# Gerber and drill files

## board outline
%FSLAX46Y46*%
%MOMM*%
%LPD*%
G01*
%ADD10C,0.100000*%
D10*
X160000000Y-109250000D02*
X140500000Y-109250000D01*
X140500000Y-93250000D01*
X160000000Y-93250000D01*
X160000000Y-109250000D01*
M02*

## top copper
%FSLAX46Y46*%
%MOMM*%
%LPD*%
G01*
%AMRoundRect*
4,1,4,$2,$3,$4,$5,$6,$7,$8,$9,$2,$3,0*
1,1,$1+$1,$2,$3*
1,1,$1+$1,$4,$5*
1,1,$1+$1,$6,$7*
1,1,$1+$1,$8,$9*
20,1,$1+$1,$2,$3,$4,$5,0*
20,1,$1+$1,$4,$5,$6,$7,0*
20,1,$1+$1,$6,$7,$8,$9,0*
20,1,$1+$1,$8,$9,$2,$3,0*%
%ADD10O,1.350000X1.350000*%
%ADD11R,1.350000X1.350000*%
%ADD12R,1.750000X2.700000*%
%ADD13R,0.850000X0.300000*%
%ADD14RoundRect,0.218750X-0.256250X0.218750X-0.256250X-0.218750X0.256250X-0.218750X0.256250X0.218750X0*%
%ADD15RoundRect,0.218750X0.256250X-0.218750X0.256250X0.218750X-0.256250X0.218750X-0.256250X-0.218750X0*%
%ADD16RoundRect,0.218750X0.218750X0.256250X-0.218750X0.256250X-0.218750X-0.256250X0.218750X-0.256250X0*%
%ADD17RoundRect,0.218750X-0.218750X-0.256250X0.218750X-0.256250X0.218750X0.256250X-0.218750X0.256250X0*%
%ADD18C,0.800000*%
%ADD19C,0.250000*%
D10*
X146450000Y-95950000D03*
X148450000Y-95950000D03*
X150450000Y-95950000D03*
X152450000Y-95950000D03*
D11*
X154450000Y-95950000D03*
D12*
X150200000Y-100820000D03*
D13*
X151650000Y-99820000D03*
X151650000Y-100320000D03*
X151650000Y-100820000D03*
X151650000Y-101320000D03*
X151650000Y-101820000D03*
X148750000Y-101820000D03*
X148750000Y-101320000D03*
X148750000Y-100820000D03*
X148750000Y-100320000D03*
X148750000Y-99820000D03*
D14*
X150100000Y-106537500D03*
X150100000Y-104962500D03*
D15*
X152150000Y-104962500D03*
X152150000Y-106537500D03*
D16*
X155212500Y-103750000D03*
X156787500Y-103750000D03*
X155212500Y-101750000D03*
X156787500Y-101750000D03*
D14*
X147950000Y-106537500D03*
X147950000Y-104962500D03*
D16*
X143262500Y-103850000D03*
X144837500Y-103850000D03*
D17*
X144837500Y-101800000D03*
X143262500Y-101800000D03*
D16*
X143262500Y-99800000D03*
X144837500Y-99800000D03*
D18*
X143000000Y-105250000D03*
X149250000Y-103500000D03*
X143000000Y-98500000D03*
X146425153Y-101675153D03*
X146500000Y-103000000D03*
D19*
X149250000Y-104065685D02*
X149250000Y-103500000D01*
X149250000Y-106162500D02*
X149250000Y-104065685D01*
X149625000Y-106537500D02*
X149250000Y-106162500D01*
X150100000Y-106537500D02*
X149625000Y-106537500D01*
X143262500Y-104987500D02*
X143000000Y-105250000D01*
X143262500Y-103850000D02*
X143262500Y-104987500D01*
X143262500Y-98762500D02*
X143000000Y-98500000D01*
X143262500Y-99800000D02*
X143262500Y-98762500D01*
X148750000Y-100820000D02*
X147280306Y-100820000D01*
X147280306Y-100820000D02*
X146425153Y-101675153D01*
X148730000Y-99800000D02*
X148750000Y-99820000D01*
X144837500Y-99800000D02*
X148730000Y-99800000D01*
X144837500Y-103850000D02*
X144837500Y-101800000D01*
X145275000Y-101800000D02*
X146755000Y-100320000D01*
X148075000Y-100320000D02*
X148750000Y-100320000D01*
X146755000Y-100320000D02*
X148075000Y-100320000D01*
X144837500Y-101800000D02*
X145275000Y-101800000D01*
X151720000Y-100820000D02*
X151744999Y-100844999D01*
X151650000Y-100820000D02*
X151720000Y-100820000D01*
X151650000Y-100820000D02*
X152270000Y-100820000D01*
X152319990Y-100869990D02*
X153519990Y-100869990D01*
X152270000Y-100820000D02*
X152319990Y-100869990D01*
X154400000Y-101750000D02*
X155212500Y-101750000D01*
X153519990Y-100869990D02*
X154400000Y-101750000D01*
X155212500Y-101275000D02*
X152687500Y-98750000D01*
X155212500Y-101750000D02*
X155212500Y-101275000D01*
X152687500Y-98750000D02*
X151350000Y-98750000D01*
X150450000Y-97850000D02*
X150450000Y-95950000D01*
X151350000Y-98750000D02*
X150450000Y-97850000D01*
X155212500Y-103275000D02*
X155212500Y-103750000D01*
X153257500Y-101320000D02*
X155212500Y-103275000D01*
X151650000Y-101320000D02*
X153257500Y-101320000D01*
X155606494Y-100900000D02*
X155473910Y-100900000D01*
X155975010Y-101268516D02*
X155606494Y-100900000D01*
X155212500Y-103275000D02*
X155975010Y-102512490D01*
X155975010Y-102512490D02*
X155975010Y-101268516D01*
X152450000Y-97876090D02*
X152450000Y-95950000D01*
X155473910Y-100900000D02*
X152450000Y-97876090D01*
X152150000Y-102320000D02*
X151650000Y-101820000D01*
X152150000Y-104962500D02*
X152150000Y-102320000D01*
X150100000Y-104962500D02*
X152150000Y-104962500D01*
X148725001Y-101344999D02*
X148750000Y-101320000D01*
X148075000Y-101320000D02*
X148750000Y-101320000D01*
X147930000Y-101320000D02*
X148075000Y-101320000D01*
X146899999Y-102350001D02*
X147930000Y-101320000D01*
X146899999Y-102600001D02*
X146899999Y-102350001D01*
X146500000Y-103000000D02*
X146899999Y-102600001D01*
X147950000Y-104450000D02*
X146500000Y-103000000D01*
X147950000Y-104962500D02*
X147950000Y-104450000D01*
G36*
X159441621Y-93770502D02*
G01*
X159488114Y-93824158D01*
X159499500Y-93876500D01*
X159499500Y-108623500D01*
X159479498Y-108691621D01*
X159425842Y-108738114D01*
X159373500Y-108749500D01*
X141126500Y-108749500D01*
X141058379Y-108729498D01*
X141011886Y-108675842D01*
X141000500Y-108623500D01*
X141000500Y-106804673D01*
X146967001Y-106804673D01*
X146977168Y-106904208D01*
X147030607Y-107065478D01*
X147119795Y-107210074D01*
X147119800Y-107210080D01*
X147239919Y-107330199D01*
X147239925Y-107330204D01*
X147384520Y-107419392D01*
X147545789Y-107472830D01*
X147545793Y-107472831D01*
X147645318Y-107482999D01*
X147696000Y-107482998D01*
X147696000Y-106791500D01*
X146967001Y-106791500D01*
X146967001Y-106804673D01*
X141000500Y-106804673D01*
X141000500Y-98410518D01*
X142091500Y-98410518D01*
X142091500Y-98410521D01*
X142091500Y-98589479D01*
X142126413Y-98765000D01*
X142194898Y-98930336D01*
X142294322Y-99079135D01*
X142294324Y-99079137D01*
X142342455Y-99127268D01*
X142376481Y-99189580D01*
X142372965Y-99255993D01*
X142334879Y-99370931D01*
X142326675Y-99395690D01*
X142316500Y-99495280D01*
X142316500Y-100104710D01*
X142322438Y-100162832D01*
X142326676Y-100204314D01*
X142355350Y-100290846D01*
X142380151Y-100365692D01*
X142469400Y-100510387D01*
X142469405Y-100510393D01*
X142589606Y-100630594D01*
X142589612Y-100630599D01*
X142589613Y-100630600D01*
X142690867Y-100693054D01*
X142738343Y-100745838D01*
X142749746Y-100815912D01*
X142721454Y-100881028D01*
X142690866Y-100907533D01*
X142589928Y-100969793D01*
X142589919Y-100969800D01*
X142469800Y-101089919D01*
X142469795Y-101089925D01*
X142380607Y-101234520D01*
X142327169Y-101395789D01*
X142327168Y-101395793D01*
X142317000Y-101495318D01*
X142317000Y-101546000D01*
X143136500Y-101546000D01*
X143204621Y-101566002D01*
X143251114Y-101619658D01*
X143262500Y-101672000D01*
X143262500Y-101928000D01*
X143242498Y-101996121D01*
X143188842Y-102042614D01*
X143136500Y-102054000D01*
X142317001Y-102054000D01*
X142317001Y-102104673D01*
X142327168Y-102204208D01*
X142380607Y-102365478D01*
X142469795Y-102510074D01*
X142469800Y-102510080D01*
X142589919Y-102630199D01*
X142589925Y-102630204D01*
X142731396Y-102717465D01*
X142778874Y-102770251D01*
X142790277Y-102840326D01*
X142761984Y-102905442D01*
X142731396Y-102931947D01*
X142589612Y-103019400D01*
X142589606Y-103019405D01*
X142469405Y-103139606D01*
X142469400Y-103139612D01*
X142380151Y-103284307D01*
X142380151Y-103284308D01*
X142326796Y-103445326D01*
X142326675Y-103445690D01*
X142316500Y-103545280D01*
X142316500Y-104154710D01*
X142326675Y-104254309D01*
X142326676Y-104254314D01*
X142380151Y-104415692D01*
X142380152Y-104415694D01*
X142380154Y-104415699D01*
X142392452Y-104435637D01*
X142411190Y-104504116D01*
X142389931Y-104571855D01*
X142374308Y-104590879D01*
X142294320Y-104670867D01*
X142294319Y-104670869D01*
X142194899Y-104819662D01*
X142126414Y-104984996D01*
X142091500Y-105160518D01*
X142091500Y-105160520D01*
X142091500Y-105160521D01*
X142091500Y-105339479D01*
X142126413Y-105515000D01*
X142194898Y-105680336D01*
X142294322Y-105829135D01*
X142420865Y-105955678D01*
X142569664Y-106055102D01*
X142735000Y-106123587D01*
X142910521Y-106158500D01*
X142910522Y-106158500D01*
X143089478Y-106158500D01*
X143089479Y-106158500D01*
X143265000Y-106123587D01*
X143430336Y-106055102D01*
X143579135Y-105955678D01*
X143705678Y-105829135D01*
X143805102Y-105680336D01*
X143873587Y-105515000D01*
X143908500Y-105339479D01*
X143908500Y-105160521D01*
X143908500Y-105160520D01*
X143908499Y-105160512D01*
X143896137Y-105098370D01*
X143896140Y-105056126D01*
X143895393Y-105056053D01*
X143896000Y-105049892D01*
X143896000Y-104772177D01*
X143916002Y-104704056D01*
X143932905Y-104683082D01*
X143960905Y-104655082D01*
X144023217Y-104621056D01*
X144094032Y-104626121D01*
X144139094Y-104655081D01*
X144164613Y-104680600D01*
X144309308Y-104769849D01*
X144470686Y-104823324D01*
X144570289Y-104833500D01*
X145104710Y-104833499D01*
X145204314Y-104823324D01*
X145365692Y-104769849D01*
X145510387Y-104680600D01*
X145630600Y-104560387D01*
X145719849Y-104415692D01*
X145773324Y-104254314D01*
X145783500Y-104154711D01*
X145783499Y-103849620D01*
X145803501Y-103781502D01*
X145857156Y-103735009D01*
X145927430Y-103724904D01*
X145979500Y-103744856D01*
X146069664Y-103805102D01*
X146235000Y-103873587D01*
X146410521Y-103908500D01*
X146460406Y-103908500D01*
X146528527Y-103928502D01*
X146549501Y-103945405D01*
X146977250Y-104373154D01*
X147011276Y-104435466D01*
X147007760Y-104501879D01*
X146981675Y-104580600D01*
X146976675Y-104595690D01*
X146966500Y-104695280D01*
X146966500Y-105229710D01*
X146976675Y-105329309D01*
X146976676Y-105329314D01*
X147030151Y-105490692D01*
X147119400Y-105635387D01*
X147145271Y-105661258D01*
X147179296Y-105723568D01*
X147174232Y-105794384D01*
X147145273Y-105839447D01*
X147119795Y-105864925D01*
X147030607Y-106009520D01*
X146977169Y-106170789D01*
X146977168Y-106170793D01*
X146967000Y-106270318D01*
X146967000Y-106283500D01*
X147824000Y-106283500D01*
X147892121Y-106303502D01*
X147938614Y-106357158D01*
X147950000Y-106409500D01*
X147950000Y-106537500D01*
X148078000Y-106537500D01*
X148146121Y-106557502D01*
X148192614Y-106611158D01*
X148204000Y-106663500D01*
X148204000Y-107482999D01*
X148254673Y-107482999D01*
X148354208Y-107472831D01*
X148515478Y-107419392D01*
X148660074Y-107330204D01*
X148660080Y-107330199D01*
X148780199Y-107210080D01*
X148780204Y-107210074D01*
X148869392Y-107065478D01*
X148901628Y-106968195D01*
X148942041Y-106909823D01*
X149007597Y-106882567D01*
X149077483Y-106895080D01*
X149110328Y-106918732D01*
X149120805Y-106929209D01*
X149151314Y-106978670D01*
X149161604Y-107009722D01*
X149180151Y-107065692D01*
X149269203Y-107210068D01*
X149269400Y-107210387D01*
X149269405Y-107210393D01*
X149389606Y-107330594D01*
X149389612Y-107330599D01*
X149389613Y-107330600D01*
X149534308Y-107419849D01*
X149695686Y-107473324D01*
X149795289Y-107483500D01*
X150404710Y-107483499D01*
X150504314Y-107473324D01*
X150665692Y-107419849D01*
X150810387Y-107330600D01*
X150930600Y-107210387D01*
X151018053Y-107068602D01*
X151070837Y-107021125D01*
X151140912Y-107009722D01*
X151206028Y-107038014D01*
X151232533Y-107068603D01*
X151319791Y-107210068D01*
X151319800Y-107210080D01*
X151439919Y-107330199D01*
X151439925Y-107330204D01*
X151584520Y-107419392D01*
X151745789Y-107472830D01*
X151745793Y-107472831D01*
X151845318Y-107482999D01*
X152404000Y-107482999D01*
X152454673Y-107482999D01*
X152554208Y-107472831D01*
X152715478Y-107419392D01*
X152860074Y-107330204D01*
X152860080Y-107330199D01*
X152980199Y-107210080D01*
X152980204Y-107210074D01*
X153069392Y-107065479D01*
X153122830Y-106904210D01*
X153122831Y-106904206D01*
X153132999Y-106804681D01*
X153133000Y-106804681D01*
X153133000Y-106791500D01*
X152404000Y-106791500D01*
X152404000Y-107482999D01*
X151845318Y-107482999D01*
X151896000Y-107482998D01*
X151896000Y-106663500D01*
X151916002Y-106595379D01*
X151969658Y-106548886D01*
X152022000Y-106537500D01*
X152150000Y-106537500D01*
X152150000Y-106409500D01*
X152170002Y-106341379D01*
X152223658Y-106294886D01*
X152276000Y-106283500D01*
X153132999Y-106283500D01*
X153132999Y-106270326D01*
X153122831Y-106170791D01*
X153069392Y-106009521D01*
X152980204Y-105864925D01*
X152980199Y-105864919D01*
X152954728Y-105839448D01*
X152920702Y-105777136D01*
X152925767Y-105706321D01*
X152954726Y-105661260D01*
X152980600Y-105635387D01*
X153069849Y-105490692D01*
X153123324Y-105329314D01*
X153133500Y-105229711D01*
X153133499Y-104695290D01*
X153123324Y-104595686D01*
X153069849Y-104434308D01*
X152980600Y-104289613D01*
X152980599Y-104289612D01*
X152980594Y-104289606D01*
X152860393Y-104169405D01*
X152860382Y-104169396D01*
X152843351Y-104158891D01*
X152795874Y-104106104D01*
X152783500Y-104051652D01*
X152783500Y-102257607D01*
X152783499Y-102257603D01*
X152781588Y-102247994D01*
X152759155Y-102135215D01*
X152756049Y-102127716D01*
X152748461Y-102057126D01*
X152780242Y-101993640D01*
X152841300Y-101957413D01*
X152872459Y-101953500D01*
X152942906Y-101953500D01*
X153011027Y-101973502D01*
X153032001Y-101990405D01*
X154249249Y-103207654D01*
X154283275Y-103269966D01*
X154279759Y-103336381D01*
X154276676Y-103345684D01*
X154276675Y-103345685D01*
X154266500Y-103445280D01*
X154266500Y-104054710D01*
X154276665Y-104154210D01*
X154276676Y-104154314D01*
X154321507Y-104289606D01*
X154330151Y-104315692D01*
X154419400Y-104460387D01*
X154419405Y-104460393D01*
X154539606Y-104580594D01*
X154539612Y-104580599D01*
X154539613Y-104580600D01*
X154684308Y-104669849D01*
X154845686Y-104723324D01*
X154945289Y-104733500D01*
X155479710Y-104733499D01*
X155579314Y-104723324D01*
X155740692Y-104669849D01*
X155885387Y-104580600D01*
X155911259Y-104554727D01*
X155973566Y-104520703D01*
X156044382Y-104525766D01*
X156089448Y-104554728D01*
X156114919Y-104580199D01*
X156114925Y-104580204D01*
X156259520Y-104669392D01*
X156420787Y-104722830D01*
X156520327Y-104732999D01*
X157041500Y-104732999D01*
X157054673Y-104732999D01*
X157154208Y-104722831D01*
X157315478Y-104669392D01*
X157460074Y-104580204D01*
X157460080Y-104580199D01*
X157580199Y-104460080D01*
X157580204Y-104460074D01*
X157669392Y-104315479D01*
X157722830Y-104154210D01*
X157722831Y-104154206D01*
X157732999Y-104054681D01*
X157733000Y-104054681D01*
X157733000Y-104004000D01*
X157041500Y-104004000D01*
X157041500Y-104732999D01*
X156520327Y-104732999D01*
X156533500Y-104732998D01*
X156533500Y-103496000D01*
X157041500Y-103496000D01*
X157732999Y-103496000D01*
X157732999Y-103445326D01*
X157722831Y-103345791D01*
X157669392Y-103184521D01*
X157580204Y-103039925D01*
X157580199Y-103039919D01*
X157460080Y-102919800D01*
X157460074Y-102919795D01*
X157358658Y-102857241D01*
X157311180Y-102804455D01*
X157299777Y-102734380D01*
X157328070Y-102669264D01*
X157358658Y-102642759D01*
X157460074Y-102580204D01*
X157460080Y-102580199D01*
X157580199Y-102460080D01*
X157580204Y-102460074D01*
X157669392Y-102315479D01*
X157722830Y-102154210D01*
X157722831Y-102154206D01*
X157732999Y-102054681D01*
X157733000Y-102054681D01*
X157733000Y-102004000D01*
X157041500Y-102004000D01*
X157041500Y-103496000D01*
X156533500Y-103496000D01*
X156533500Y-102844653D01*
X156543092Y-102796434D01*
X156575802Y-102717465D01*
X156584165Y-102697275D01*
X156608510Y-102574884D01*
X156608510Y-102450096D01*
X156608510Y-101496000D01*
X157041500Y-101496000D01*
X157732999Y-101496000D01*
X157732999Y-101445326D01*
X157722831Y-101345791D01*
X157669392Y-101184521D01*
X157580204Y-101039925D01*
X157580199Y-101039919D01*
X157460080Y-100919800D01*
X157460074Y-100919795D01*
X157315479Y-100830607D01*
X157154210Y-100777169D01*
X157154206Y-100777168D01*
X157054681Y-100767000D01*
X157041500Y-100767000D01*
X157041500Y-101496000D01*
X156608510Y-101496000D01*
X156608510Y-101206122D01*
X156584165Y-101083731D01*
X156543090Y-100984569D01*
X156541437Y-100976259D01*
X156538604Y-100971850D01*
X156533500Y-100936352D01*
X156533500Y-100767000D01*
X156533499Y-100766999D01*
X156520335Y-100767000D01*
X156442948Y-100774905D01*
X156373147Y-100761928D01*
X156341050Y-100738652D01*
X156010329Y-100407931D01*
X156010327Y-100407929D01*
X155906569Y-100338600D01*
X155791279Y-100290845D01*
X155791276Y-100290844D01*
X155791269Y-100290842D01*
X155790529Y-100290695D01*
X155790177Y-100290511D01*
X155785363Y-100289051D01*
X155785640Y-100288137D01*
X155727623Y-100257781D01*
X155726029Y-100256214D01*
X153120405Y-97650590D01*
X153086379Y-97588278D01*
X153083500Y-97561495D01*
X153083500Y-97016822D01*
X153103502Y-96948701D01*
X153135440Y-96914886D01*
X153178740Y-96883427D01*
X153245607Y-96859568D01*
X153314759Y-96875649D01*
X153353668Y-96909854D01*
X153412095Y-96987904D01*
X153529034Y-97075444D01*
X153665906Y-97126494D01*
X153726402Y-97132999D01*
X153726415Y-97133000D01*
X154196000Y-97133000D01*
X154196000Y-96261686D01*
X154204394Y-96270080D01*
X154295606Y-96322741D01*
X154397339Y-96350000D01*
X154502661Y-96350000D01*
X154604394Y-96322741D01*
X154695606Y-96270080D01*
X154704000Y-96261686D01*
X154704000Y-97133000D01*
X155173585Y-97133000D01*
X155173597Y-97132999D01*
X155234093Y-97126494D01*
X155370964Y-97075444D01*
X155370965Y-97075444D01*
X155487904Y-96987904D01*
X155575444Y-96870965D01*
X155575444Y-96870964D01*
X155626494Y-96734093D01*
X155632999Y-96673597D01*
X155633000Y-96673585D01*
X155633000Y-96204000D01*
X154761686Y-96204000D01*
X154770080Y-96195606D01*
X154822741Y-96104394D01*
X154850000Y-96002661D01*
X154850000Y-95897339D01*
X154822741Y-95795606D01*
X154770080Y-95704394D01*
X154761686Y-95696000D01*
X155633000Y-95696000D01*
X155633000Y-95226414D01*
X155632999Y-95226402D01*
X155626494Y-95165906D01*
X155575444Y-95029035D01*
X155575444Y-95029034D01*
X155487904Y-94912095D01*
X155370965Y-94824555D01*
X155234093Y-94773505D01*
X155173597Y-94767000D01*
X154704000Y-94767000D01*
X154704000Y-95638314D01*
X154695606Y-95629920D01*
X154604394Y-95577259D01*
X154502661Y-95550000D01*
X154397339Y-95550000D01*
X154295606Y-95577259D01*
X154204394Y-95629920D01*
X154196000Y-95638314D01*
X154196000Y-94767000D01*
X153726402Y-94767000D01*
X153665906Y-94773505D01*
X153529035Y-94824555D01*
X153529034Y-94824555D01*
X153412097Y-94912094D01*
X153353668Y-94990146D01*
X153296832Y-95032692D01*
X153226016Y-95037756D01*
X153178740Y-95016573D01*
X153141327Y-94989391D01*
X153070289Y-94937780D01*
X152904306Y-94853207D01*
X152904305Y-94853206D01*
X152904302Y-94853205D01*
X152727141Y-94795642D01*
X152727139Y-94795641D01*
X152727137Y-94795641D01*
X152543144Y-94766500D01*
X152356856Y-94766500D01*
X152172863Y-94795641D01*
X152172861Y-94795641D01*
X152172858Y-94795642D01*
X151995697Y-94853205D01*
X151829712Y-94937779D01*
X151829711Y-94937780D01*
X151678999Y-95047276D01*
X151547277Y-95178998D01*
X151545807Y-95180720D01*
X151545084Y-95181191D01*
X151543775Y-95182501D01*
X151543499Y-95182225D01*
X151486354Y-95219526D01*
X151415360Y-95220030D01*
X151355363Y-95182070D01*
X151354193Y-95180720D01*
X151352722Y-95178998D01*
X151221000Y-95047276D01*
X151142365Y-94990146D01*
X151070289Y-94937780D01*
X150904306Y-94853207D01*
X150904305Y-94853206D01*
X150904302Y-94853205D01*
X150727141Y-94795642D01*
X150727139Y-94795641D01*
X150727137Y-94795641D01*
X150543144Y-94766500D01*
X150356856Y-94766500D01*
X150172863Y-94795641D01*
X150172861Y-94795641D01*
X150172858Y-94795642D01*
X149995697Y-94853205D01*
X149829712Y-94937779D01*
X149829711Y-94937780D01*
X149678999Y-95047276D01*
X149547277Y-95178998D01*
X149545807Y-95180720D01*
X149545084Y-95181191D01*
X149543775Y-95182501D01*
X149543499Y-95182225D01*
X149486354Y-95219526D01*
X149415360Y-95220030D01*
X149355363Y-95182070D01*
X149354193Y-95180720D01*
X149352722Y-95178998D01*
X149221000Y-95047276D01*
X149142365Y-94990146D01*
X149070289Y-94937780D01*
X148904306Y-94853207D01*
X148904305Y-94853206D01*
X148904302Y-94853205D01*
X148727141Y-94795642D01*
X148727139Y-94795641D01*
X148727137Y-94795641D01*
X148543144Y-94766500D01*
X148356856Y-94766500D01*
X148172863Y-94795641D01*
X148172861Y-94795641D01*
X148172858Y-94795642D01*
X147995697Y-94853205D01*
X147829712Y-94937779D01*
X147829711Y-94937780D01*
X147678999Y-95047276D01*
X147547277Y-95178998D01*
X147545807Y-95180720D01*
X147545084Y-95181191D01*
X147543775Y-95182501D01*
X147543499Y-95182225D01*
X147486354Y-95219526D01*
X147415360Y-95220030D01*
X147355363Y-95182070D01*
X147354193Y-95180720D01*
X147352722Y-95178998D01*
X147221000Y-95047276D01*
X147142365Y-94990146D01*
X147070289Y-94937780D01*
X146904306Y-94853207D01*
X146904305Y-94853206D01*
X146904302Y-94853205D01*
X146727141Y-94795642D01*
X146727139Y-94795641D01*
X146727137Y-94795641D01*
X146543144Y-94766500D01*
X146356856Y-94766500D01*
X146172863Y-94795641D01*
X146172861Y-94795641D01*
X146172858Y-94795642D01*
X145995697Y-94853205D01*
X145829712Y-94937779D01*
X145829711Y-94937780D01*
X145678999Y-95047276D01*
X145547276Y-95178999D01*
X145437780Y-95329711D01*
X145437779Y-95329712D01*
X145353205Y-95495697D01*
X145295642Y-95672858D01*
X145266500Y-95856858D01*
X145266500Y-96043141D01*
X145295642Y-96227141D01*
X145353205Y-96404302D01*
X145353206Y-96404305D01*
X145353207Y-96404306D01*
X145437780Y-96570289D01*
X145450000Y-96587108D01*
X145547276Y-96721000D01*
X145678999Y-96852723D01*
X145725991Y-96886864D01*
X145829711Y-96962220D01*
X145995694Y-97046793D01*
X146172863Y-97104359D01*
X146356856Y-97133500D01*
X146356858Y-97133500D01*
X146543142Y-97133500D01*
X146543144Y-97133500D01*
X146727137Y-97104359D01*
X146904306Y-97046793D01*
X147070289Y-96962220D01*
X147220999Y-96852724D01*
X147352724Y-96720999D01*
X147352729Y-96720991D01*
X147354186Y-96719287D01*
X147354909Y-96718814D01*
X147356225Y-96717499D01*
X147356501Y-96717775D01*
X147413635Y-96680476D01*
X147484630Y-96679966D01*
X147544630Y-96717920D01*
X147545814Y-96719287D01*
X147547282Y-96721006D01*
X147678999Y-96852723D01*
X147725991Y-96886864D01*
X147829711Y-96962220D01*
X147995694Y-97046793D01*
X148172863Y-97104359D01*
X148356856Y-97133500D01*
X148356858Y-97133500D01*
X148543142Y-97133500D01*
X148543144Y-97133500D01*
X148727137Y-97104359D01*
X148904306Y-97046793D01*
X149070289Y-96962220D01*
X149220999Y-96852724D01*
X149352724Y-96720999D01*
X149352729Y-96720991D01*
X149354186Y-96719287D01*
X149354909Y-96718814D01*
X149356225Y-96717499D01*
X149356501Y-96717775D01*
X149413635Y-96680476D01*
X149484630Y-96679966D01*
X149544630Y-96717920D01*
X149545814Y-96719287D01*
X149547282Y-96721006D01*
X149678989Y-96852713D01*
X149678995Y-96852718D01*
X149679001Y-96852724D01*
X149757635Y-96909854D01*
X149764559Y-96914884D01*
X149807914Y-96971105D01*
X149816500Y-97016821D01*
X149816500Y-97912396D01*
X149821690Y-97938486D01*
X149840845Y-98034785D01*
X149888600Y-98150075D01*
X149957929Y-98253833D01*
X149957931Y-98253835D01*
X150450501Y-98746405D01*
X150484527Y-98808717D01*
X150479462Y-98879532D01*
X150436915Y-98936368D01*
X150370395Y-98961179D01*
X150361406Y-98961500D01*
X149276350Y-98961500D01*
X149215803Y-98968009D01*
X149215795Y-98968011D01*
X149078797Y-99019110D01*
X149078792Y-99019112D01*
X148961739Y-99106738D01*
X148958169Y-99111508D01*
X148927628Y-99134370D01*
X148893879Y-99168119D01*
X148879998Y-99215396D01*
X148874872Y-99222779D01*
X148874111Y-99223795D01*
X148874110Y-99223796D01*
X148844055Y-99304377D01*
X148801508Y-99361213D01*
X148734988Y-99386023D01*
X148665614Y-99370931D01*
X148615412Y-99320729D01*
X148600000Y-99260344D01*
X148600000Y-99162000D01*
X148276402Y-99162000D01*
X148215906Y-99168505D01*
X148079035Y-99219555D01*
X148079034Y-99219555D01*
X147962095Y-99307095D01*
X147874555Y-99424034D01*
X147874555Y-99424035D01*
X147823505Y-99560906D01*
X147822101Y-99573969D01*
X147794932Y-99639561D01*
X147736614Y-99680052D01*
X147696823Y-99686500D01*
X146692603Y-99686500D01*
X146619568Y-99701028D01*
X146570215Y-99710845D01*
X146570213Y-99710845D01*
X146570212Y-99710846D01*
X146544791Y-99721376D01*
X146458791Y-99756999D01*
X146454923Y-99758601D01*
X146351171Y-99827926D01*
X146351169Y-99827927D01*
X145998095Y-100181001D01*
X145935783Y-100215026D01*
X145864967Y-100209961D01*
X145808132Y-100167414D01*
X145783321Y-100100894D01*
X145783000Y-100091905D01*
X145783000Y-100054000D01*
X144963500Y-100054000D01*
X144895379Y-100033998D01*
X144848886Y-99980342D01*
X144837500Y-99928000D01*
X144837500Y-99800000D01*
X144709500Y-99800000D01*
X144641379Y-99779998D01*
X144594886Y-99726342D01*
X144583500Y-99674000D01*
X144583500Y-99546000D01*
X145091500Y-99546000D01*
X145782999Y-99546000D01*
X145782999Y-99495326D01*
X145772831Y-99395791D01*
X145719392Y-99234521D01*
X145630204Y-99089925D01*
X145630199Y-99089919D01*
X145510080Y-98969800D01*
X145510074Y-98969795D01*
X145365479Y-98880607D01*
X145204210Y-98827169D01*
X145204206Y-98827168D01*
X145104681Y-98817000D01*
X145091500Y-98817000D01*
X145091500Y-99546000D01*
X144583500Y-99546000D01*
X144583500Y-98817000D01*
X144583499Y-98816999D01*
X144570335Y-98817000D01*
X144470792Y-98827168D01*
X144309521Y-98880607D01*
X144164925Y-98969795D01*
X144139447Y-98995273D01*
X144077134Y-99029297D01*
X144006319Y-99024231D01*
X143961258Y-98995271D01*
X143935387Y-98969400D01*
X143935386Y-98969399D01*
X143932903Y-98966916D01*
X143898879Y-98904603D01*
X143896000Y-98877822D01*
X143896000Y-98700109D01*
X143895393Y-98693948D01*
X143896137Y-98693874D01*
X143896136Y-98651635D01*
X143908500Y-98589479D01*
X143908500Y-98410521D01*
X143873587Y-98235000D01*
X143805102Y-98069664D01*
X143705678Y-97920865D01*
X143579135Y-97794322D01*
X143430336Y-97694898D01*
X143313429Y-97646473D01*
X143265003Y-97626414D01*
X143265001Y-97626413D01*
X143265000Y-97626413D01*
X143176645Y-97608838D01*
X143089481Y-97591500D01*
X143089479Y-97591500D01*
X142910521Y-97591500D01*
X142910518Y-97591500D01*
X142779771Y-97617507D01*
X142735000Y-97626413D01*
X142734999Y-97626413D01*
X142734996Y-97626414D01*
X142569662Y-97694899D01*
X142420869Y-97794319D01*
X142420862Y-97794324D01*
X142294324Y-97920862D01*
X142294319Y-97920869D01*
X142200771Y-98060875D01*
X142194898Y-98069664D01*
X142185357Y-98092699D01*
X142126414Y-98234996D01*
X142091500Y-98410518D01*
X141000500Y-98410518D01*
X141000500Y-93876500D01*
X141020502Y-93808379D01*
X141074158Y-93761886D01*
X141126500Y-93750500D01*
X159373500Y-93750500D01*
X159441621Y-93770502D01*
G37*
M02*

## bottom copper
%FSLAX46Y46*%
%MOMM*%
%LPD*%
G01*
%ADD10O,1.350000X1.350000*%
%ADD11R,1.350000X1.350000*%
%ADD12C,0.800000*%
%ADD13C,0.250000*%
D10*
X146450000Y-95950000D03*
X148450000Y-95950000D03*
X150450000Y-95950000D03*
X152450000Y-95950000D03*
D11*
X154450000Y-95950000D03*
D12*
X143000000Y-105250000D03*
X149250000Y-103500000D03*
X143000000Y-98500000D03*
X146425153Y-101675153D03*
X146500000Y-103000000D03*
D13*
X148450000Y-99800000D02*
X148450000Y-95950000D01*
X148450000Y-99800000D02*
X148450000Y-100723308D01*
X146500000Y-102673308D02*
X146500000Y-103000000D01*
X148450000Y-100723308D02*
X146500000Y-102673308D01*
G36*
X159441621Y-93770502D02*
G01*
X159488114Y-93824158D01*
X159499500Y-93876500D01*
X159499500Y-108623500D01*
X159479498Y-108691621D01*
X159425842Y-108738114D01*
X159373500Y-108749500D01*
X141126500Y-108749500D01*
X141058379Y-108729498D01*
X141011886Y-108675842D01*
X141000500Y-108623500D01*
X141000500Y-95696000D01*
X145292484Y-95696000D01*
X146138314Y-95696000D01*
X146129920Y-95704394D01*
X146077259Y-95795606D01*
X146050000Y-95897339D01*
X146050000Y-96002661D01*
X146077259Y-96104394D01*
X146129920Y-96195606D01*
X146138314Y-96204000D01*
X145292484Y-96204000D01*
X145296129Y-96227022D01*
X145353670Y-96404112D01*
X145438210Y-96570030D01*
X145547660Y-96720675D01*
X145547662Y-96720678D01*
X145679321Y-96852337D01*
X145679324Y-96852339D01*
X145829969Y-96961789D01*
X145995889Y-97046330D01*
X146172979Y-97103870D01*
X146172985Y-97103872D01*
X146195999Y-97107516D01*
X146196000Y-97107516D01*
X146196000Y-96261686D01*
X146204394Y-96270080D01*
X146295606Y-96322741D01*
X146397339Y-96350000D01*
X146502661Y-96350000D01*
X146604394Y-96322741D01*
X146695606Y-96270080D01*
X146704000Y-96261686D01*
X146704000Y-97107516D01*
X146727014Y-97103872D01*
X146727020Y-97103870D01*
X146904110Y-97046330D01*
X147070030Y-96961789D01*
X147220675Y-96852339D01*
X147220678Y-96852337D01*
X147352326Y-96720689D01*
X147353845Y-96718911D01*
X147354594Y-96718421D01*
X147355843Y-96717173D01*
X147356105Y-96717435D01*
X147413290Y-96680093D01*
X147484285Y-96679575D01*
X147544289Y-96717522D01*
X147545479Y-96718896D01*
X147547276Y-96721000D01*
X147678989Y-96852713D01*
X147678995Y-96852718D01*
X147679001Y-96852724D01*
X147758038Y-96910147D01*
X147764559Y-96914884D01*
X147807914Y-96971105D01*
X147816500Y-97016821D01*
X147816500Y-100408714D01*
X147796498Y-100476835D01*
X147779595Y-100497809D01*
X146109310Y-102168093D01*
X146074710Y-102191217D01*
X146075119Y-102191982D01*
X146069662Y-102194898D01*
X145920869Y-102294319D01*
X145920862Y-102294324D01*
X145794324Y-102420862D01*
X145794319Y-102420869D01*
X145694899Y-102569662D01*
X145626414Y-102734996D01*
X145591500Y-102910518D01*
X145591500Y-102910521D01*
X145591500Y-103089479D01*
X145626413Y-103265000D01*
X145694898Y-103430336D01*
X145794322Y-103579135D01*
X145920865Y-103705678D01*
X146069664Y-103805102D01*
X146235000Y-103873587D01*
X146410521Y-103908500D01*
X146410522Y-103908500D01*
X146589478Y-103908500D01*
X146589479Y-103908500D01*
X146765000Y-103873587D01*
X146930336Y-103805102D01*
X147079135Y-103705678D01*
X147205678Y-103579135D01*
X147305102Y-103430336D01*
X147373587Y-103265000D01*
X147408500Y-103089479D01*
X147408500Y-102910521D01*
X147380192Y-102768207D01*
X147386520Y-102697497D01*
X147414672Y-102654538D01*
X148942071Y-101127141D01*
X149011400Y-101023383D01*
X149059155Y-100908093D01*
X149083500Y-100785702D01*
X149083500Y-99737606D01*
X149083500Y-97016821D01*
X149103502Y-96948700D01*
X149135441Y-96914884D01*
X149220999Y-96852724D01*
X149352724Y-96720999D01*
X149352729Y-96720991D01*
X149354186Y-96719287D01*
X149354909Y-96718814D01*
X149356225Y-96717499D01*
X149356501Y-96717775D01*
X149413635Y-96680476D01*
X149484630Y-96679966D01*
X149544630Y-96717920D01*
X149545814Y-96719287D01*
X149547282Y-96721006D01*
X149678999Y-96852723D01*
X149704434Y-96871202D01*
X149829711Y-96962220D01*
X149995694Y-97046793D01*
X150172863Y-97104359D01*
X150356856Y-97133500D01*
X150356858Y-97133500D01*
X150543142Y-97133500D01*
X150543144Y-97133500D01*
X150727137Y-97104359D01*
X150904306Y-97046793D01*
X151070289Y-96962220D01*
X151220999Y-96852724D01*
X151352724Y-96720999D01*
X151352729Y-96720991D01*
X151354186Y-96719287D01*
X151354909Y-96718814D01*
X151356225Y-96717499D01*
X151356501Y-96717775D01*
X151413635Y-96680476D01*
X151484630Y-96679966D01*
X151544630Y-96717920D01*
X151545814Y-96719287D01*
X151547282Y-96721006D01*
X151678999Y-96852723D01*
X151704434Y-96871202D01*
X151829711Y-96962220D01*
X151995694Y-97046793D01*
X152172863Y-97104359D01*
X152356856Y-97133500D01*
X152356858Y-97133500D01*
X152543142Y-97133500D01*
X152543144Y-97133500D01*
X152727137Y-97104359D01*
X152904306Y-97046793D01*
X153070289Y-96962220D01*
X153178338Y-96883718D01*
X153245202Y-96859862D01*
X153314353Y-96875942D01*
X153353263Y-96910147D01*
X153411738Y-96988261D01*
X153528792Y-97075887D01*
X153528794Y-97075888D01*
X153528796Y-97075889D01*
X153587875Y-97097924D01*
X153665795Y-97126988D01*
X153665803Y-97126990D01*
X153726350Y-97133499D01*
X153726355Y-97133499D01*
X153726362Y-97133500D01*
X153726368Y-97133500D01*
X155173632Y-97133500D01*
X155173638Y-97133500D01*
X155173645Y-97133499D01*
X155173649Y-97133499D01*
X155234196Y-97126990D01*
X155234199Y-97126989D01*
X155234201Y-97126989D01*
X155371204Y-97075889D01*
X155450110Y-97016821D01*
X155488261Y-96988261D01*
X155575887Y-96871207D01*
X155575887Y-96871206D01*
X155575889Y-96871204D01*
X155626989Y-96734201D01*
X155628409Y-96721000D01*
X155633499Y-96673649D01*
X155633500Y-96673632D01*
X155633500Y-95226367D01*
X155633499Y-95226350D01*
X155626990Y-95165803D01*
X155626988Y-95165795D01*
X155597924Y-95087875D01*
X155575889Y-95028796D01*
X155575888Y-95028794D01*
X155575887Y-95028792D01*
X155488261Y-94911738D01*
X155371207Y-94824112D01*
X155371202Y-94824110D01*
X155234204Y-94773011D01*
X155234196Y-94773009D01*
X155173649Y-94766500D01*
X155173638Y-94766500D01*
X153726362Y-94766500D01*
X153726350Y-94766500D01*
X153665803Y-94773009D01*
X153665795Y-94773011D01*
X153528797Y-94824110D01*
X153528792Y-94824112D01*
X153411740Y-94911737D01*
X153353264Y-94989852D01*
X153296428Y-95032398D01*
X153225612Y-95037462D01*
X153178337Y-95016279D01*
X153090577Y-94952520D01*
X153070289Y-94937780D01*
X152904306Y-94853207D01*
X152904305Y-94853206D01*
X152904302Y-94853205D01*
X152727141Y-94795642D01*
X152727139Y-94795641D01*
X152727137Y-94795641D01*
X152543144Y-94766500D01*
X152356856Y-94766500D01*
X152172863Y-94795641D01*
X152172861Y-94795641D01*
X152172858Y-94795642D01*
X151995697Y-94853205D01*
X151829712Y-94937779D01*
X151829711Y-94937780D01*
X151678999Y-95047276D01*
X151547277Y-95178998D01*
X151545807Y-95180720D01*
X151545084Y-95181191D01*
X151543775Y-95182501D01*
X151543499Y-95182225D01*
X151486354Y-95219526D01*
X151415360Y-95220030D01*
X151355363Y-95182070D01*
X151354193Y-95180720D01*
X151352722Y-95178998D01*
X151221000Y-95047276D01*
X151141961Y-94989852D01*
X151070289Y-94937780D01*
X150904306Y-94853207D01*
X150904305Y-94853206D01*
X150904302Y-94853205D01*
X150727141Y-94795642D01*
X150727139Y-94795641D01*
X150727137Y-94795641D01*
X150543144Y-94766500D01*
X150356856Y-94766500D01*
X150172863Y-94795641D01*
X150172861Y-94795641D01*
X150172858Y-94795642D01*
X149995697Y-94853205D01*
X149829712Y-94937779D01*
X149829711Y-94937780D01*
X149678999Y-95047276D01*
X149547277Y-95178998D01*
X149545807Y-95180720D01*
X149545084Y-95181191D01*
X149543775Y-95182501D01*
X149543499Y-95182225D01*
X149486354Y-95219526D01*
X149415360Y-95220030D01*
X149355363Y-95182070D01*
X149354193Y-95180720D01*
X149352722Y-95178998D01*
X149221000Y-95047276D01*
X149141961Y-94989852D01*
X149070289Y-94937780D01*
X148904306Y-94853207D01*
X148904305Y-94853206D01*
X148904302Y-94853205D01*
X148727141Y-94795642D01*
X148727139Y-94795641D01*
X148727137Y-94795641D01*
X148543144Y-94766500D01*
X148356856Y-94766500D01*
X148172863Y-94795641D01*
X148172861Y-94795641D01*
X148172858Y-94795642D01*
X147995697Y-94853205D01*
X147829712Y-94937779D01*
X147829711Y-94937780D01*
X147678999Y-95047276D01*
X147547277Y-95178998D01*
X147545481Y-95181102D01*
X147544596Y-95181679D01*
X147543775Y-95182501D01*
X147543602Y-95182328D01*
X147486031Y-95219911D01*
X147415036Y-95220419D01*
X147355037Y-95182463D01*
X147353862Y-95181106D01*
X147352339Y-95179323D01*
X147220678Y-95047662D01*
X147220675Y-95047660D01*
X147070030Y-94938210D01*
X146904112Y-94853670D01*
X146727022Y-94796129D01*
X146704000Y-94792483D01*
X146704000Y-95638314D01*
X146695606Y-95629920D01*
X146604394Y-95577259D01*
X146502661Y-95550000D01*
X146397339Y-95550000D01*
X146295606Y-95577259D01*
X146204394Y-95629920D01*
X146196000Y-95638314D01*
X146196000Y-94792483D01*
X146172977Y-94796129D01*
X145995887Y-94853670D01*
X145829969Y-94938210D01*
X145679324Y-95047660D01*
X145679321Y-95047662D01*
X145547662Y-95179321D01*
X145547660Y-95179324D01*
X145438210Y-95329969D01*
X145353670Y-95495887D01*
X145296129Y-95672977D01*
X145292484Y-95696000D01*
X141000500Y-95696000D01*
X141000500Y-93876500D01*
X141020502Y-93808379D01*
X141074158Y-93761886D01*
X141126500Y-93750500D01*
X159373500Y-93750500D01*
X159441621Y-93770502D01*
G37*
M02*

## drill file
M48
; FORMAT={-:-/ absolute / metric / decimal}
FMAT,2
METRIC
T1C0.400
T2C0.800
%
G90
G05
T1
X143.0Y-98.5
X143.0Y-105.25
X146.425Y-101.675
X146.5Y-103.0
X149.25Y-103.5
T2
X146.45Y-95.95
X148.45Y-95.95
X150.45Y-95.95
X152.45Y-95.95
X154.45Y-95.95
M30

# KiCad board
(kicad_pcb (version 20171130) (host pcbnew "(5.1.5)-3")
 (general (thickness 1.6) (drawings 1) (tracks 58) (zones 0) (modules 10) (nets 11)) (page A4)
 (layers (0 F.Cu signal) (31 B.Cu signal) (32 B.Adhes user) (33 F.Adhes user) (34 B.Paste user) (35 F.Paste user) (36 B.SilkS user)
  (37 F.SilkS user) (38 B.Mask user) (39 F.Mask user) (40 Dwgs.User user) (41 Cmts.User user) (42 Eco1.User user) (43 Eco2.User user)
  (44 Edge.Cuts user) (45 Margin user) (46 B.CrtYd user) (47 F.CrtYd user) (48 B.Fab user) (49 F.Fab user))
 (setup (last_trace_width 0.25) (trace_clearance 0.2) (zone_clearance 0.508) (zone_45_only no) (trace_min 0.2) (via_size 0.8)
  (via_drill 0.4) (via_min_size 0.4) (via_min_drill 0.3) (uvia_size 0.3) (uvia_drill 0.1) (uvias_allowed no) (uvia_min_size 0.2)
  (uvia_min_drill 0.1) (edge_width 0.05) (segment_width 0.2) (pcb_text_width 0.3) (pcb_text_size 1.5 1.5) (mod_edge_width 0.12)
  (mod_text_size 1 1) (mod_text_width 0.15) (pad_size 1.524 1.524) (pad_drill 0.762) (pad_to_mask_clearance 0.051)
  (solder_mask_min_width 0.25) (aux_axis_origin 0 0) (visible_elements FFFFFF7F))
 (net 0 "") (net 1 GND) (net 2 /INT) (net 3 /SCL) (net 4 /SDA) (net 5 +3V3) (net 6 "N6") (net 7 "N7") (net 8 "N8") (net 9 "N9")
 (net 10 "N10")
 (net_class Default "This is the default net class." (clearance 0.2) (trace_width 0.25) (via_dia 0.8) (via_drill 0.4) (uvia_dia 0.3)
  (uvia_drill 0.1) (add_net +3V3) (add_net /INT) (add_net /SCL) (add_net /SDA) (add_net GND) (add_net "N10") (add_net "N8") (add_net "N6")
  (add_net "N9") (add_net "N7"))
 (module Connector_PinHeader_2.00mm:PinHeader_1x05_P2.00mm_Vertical (layer F.Cu) (at 154.45 95.95 270)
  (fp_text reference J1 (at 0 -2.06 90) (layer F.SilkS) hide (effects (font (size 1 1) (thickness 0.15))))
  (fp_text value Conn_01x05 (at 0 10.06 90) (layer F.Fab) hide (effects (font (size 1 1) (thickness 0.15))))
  (pad 5 thru_hole oval (at 0 8 270) (size 1.35 1.35) (drill 0.8) (layers *.Cu *.Mask) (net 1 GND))
  (pad 4 thru_hole oval (at 0 6 270) (size 1.35 1.35) (drill 0.8) (layers *.Cu *.Mask) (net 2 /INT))
  (pad 3 thru_hole oval (at 0 4 270) (size 1.35 1.35) (drill 0.8) (layers *.Cu *.Mask) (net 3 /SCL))
  (pad 2 thru_hole oval (at 0 2 270) (size 1.35 1.35) (drill 0.8) (layers *.Cu *.Mask) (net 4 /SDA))
  (pad 1 thru_hole rect (at 0 0 270) (size 1.35 1.35) (drill 0.8) (layers *.Cu *.Mask) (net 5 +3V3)))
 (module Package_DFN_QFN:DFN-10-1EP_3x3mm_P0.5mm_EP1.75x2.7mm (layer F.Cu) (at 150.2 100.82)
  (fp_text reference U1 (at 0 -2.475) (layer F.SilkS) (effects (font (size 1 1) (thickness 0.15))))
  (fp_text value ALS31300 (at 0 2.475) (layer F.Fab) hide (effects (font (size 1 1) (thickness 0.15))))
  (pad "" smd rect (at 0.3875 0.62) (size 0.6 1.05) (layers F.Paste))
  (pad "" smd rect (at 0.3875 -0.62) (size 0.6 1.05) (layers F.Paste))
  (pad "" smd rect (at -0.3875 0.62) (size 0.6 1.05) (layers F.Paste))
  (pad "" smd rect (at -0.3875 -0.62) (size 0.6 1.05) (layers F.Paste))
  (pad 11 smd rect (at 0 0) (size 1.75 2.7) (layers F.Cu F.Mask))
  (pad 10 smd rect (at 1.45 -1) (size 0.85 0.3) (layers F.Cu F.Paste F.Mask) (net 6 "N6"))
  (pad 9 smd rect (at 1.45 -0.5) (size 0.85 0.3) (layers F.Cu F.Paste F.Mask) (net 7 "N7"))
  (pad 8 smd rect (at 1.45 0) (size 0.85 0.3) (layers F.Cu F.Paste F.Mask) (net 3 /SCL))
  (pad 7 smd rect (at 1.45 0.5) (size 0.85 0.3) (layers F.Cu F.Paste F.Mask) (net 4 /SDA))
  (pad 6 smd rect (at 1.45 1) (size 0.85 0.3) (layers F.Cu F.Paste F.Mask) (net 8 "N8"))
  (pad 5 smd rect (at -1.45 1) (size 0.85 0.3) (layers F.Cu F.Paste F.Mask) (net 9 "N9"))
  (pad 4 smd rect (at -1.45 0.5) (size 0.85 0.3) (layers F.Cu F.Paste F.Mask) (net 2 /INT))
  (pad 3 smd rect (at -1.45 0) (size 0.85 0.3) (layers F.Cu F.Paste F.Mask) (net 1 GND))
  (pad 2 smd rect (at -1.45 -0.5) (size 0.85 0.3) (layers F.Cu F.Paste F.Mask) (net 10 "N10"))
  (pad 1 smd rect (at -1.45 -1) (size 0.85 0.3) (layers F.Cu F.Paste F.Mask) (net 5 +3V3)))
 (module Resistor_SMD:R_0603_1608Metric (layer F.Cu) (at 150.1 105.75 270)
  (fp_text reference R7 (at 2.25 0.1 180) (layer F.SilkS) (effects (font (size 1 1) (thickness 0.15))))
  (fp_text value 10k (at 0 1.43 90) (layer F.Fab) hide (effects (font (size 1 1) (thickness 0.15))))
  (pad 2 smd roundrect (at 0.7875 0 270) (size 0.875 0.95) (layers F.Cu F.Paste F.Mask) (roundrect_rratio 0.25) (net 1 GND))
  (pad 1 smd roundrect (at -0.7875 0 270) (size 0.875 0.95) (layers F.Cu F.Paste F.Mask) (roundrect_rratio 0.25) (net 8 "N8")))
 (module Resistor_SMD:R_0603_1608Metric (layer F.Cu) (at 152.15 105.75 90)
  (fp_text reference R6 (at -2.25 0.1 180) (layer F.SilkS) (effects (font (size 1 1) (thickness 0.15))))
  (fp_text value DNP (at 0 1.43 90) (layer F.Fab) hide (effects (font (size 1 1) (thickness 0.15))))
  (pad 2 smd roundrect (at 0.7875 0 90) (size 0.875 0.95) (layers F.Cu F.Paste F.Mask) (roundrect_rratio 0.25) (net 8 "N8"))
  (pad 1 smd roundrect (at -0.7875 0 90) (size 0.875 0.95) (layers F.Cu F.Paste F.Mask) (roundrect_rratio 0.25) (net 5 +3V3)))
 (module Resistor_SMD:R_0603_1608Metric (layer F.Cu) (at 156 103.75 180)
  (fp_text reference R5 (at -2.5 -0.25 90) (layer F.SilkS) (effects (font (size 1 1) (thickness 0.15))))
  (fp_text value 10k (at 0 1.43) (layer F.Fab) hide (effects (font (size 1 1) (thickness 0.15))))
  (pad 2 smd roundrect (at 0.7875 0 180) (size 0.875 0.95) (layers F.Cu F.Paste F.Mask) (roundrect_rratio 0.25) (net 4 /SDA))
  (pad 1 smd roundrect (at -0.7875 0 180) (size 0.875 0.95) (layers F.Cu F.Paste F.Mask) (roundrect_rratio 0.25) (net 5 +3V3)))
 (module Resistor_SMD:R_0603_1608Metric (layer F.Cu) (at 156 101.75 180)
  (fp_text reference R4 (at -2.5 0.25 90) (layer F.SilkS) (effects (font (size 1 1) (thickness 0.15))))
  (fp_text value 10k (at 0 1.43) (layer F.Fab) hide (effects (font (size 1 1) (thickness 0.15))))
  (pad 2 smd roundrect (at 0.7875 0 180) (size 0.875 0.95) (layers F.Cu F.Paste F.Mask) (roundrect_rratio 0.25) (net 3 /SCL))
  (pad 1 smd roundrect (at -0.7875 0 180) (size 0.875 0.95) (layers F.Cu F.Paste F.Mask) (roundrect_rratio 0.25) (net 5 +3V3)))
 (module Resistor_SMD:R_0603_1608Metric (layer F.Cu) (at 147.95 105.75 270)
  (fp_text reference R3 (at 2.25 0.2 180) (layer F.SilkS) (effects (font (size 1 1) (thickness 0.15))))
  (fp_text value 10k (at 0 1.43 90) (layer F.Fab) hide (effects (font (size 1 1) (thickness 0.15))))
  (pad 2 smd roundrect (at 0.7875 0 270) (size 0.875 0.95) (layers F.Cu F.Paste F.Mask) (roundrect_rratio 0.25) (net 5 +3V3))
  (pad 1 smd roundrect (at -0.7875 0 270) (size 0.875 0.95) (layers F.Cu F.Paste F.Mask) (roundrect_rratio 0.25) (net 2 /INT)))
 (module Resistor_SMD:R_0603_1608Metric (layer F.Cu) (at 144.05 103.85 180)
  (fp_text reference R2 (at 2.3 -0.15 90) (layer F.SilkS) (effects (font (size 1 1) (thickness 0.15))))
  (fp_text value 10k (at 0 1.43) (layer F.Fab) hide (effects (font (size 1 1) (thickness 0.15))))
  (pad 2 smd roundrect (at 0.7875 0 180) (size 0.875 0.95) (layers F.Cu F.Paste F.Mask) (roundrect_rratio 0.25) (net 1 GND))
  (pad 1 smd roundrect (at -0.7875 0 180) (size 0.875 0.95) (layers F.Cu F.Paste F.Mask) (roundrect_rratio 0.25) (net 10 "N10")))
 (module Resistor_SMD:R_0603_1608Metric (layer F.Cu) (at 144.05 101.8)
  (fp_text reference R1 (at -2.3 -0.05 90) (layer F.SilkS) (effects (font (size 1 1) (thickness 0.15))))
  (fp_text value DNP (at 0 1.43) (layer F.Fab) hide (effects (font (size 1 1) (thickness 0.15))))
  (pad 2 smd roundrect (at 0.7875 0) (size 0.875 0.95) (layers F.Cu F.Paste F.Mask) (roundrect_rratio 0.25) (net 10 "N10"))
  (pad 1 smd roundrect (at -0.7875 0) (size 0.875 0.95) (layers F.Cu F.Paste F.Mask) (roundrect_rratio 0.25) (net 5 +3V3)))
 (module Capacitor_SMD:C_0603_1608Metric (layer F.Cu) (at 144.05 99.8 180)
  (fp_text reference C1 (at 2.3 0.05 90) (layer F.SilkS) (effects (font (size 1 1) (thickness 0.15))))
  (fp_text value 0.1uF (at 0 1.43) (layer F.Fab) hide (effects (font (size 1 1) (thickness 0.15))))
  (pad 2 smd roundrect (at 0.7875 0 180) (size 0.875 0.95) (layers F.Cu F.Paste F.Mask) (roundrect_rratio 0.25) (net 1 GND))
  (pad 1 smd roundrect (at -0.7875 0 180) (size 0.875 0.95) (layers F.Cu F.Paste F.Mask) (roundrect_rratio 0.25) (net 5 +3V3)))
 (gr_poly (pts (xy 160 109.25) (xy 140.5 109.25) (xy 140.5 93.25) (xy 160 93.25)) (layer Edge.Cuts) (width 0.1))
 (via (at 143 105.25) (size 0.8) (drill 0.4) (layers F.Cu B.Cu) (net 1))
 (via (at 149.25 103.5) (size 0.8) (drill 0.4) (layers F.Cu B.Cu) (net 1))
 (via (at 143 98.5) (size 0.8) (drill 0.4) (layers F.Cu B.Cu) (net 1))
 (segment (start 149.25 104.065685) (end 149.25 103.5) (width 0.25) (layer F.Cu) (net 1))
 (segment (start 149.25 106.1625) (end 149.25 104.065685) (width 0.25) (layer F.Cu) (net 1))
 (segment (start 149.625 106.5375) (end 149.25 106.1625) (width 0.25) (layer F.Cu) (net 1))
 (segment (start 150.1 106.5375) (end 149.625 106.5375) (width 0.25) (layer F.Cu) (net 1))
 (segment (start 143.2625 104.9875) (end 143 105.25) (width 0.25) (layer F.Cu) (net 1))
 (segment (start 143.2625 103.85) (end 143.2625 104.9875) (width 0.25) (layer F.Cu) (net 1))
 (segment (start 143.2625 98.7625) (end 143 98.5) (width 0.25) (layer F.Cu) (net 1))
 (segment (start 143.2625 99.8) (end 143.2625 98.7625) (width 0.25) (layer F.Cu) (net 1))
 (via (at 146.425153 101.675153) (size 0.8) (drill 0.4) (layers F.Cu B.Cu) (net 1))
 (segment (start 148.75 100.82) (end 147.280306 100.82) (width 0.25) (layer F.Cu) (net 1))
 (segment (start 147.280306 100.82) (end 146.425153 101.675153) (width 0.25) (layer F.Cu) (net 1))
 (segment (start 148.73 99.8) (end 148.75 99.82) (width 0.25) (layer F.Cu) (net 5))
 (segment (start 144.8375 99.8) (end 148.73 99.8) (width 0.25) (layer F.Cu) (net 5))
 (segment (start 144.8375 103.85) (end 144.8375 101.8) (width 0.25) (layer F.Cu) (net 10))
 (segment (start 145.275 101.8) (end 146.755 100.32) (width 0.25) (layer F.Cu) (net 10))
 (segment (start 148.075 100.32) (end 148.75 100.32) (width 0.25) (layer F.Cu) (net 10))
 (segment (start 146.755 100.32) (end 148.075 100.32) (width 0.25) (layer F.Cu) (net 10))
 (segment (start 144.8375 101.8) (end 145.275 101.8) (width 0.25) (layer F.Cu) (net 10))
 (segment (start 151.72 100.82) (end 151.744999 100.844999) (width 0.25) (layer F.Cu) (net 3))
 (segment (start 151.65 100.82) (end 151.72 100.82) (width 0.25) (layer F.Cu) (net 3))
 (segment (start 151.65 100.82) (end 152.27 100.82) (width 0.25) (layer F.Cu) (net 3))
 (segment (start 152.31999 100.86999) (end 153.51999 100.86999) (width 0.25) (layer F.Cu) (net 3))
 (segment (start 152.27 100.82) (end 152.31999 100.86999) (width 0.25) (layer F.Cu) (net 3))
 (segment (start 154.4 101.75) (end 155.2125 101.75) (width 0.25) (layer F.Cu) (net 3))
 (segment (start 153.51999 100.86999) (end 154.4 101.75) (width 0.25) (layer F.Cu) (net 3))
 (segment (start 155.2125 101.275) (end 152.6875 98.75) (width 0.25) (layer F.Cu) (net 3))
 (segment (start 155.2125 101.75) (end 155.2125 101.275) (width 0.25) (layer F.Cu) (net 3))
 (segment (start 152.6875 98.75) (end 151.35 98.75) (width 0.25) (layer F.Cu) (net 3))
 (segment (start 150.45 97.85) (end 150.45 95.95) (width 0.25) (layer F.Cu) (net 3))
 (segment (start 151.35 98.75) (end 150.45 97.85) (width 0.25) (layer F.Cu) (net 3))
 (segment (start 155.2125 103.275) (end 155.2125 103.75) (width 0.25) (layer F.Cu) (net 4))
 (segment (start 153.2575 101.32) (end 155.2125 103.275) (width 0.25) (layer F.Cu) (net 4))
 (segment (start 151.65 101.32) (end 153.2575 101.32) (width 0.25) (layer F.Cu) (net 4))
 (segment (start 155.606494 100.9) (end 155.47391 100.9) (width 0.25) (layer F.Cu) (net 4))
 (segment (start 155.97501 101.268516) (end 155.606494 100.9) (width 0.25) (layer F.Cu) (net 4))
 (segment (start 155.2125 103.275) (end 155.97501 102.51249) (width 0.25) (layer F.Cu) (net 4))
 (segment (start 155.97501 102.51249) (end 155.97501 101.268516) (width 0.25) (layer F.Cu) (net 4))
 (segment (start 152.45 97.87609) (end 152.45 95.95) (width 0.25) (layer F.Cu) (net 4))
 (segment (start 155.47391 100.9) (end 152.45 97.87609) (width 0.25) (layer F.Cu) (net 4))
 (segment (start 152.15 102.32) (end 151.65 101.82) (width 0.25) (layer F.Cu) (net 8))
 (segment (start 152.15 104.9625) (end 152.15 102.32) (width 0.25) (layer F.Cu) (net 8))
 (segment (start 150.1 104.9625) (end 152.15 104.9625) (width 0.25) (layer F.Cu) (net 8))
 (segment (start 148.725001 101.344999) (end 148.75 101.32) (width 0.25) (layer F.Cu) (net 2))
 (segment (start 148.45 99.8) (end 148.45 95.95) (width 0.25) (layer B.Cu) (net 2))
 (via (at 146.5 103) (size 0.8) (drill 0.4) (layers F.Cu B.Cu) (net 2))
 (segment (start 148.45 99.8) (end 148.45 100.723308) (width 0.25) (layer B.Cu) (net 2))
 (segment (start 146.5 102.673308) (end 146.5 103) (width 0.25) (layer B.Cu) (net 2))
 (segment (start 148.45 100.723308) (end 146.5 102.673308) (width 0.25) (layer B.Cu) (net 2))
 (segment (start 148.075 101.32) (end 148.75 101.32) (width 0.25) (layer F.Cu) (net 2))
 (segment (start 147.93 101.32) (end 148.075 101.32) (width 0.25) (layer F.Cu) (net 2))
 (segment (start 146.899999 102.350001) (end 147.93 101.32) (width 0.25) (layer F.Cu) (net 2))
 (segment (start 146.899999 102.600001) (end 146.899999 102.350001) (width 0.25) (layer F.Cu) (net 2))
 (segment (start 146.5 103) (end 146.899999 102.600001) (width 0.25) (layer F.Cu) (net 2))
 (segment (start 147.95 104.45) (end 146.5 103) (width 0.25) (layer F.Cu) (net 2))
 (segment (start 147.95 104.9625) (end 147.95 104.45) (width 0.25) (layer F.Cu) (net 2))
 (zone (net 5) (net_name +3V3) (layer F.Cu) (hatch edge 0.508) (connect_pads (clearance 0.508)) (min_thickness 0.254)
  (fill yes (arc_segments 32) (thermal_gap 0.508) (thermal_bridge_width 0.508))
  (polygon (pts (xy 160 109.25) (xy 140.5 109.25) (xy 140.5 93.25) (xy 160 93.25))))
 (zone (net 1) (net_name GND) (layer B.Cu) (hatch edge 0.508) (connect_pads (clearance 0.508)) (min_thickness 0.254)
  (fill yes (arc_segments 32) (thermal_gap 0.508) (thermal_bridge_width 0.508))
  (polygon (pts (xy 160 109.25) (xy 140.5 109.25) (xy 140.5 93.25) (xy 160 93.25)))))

